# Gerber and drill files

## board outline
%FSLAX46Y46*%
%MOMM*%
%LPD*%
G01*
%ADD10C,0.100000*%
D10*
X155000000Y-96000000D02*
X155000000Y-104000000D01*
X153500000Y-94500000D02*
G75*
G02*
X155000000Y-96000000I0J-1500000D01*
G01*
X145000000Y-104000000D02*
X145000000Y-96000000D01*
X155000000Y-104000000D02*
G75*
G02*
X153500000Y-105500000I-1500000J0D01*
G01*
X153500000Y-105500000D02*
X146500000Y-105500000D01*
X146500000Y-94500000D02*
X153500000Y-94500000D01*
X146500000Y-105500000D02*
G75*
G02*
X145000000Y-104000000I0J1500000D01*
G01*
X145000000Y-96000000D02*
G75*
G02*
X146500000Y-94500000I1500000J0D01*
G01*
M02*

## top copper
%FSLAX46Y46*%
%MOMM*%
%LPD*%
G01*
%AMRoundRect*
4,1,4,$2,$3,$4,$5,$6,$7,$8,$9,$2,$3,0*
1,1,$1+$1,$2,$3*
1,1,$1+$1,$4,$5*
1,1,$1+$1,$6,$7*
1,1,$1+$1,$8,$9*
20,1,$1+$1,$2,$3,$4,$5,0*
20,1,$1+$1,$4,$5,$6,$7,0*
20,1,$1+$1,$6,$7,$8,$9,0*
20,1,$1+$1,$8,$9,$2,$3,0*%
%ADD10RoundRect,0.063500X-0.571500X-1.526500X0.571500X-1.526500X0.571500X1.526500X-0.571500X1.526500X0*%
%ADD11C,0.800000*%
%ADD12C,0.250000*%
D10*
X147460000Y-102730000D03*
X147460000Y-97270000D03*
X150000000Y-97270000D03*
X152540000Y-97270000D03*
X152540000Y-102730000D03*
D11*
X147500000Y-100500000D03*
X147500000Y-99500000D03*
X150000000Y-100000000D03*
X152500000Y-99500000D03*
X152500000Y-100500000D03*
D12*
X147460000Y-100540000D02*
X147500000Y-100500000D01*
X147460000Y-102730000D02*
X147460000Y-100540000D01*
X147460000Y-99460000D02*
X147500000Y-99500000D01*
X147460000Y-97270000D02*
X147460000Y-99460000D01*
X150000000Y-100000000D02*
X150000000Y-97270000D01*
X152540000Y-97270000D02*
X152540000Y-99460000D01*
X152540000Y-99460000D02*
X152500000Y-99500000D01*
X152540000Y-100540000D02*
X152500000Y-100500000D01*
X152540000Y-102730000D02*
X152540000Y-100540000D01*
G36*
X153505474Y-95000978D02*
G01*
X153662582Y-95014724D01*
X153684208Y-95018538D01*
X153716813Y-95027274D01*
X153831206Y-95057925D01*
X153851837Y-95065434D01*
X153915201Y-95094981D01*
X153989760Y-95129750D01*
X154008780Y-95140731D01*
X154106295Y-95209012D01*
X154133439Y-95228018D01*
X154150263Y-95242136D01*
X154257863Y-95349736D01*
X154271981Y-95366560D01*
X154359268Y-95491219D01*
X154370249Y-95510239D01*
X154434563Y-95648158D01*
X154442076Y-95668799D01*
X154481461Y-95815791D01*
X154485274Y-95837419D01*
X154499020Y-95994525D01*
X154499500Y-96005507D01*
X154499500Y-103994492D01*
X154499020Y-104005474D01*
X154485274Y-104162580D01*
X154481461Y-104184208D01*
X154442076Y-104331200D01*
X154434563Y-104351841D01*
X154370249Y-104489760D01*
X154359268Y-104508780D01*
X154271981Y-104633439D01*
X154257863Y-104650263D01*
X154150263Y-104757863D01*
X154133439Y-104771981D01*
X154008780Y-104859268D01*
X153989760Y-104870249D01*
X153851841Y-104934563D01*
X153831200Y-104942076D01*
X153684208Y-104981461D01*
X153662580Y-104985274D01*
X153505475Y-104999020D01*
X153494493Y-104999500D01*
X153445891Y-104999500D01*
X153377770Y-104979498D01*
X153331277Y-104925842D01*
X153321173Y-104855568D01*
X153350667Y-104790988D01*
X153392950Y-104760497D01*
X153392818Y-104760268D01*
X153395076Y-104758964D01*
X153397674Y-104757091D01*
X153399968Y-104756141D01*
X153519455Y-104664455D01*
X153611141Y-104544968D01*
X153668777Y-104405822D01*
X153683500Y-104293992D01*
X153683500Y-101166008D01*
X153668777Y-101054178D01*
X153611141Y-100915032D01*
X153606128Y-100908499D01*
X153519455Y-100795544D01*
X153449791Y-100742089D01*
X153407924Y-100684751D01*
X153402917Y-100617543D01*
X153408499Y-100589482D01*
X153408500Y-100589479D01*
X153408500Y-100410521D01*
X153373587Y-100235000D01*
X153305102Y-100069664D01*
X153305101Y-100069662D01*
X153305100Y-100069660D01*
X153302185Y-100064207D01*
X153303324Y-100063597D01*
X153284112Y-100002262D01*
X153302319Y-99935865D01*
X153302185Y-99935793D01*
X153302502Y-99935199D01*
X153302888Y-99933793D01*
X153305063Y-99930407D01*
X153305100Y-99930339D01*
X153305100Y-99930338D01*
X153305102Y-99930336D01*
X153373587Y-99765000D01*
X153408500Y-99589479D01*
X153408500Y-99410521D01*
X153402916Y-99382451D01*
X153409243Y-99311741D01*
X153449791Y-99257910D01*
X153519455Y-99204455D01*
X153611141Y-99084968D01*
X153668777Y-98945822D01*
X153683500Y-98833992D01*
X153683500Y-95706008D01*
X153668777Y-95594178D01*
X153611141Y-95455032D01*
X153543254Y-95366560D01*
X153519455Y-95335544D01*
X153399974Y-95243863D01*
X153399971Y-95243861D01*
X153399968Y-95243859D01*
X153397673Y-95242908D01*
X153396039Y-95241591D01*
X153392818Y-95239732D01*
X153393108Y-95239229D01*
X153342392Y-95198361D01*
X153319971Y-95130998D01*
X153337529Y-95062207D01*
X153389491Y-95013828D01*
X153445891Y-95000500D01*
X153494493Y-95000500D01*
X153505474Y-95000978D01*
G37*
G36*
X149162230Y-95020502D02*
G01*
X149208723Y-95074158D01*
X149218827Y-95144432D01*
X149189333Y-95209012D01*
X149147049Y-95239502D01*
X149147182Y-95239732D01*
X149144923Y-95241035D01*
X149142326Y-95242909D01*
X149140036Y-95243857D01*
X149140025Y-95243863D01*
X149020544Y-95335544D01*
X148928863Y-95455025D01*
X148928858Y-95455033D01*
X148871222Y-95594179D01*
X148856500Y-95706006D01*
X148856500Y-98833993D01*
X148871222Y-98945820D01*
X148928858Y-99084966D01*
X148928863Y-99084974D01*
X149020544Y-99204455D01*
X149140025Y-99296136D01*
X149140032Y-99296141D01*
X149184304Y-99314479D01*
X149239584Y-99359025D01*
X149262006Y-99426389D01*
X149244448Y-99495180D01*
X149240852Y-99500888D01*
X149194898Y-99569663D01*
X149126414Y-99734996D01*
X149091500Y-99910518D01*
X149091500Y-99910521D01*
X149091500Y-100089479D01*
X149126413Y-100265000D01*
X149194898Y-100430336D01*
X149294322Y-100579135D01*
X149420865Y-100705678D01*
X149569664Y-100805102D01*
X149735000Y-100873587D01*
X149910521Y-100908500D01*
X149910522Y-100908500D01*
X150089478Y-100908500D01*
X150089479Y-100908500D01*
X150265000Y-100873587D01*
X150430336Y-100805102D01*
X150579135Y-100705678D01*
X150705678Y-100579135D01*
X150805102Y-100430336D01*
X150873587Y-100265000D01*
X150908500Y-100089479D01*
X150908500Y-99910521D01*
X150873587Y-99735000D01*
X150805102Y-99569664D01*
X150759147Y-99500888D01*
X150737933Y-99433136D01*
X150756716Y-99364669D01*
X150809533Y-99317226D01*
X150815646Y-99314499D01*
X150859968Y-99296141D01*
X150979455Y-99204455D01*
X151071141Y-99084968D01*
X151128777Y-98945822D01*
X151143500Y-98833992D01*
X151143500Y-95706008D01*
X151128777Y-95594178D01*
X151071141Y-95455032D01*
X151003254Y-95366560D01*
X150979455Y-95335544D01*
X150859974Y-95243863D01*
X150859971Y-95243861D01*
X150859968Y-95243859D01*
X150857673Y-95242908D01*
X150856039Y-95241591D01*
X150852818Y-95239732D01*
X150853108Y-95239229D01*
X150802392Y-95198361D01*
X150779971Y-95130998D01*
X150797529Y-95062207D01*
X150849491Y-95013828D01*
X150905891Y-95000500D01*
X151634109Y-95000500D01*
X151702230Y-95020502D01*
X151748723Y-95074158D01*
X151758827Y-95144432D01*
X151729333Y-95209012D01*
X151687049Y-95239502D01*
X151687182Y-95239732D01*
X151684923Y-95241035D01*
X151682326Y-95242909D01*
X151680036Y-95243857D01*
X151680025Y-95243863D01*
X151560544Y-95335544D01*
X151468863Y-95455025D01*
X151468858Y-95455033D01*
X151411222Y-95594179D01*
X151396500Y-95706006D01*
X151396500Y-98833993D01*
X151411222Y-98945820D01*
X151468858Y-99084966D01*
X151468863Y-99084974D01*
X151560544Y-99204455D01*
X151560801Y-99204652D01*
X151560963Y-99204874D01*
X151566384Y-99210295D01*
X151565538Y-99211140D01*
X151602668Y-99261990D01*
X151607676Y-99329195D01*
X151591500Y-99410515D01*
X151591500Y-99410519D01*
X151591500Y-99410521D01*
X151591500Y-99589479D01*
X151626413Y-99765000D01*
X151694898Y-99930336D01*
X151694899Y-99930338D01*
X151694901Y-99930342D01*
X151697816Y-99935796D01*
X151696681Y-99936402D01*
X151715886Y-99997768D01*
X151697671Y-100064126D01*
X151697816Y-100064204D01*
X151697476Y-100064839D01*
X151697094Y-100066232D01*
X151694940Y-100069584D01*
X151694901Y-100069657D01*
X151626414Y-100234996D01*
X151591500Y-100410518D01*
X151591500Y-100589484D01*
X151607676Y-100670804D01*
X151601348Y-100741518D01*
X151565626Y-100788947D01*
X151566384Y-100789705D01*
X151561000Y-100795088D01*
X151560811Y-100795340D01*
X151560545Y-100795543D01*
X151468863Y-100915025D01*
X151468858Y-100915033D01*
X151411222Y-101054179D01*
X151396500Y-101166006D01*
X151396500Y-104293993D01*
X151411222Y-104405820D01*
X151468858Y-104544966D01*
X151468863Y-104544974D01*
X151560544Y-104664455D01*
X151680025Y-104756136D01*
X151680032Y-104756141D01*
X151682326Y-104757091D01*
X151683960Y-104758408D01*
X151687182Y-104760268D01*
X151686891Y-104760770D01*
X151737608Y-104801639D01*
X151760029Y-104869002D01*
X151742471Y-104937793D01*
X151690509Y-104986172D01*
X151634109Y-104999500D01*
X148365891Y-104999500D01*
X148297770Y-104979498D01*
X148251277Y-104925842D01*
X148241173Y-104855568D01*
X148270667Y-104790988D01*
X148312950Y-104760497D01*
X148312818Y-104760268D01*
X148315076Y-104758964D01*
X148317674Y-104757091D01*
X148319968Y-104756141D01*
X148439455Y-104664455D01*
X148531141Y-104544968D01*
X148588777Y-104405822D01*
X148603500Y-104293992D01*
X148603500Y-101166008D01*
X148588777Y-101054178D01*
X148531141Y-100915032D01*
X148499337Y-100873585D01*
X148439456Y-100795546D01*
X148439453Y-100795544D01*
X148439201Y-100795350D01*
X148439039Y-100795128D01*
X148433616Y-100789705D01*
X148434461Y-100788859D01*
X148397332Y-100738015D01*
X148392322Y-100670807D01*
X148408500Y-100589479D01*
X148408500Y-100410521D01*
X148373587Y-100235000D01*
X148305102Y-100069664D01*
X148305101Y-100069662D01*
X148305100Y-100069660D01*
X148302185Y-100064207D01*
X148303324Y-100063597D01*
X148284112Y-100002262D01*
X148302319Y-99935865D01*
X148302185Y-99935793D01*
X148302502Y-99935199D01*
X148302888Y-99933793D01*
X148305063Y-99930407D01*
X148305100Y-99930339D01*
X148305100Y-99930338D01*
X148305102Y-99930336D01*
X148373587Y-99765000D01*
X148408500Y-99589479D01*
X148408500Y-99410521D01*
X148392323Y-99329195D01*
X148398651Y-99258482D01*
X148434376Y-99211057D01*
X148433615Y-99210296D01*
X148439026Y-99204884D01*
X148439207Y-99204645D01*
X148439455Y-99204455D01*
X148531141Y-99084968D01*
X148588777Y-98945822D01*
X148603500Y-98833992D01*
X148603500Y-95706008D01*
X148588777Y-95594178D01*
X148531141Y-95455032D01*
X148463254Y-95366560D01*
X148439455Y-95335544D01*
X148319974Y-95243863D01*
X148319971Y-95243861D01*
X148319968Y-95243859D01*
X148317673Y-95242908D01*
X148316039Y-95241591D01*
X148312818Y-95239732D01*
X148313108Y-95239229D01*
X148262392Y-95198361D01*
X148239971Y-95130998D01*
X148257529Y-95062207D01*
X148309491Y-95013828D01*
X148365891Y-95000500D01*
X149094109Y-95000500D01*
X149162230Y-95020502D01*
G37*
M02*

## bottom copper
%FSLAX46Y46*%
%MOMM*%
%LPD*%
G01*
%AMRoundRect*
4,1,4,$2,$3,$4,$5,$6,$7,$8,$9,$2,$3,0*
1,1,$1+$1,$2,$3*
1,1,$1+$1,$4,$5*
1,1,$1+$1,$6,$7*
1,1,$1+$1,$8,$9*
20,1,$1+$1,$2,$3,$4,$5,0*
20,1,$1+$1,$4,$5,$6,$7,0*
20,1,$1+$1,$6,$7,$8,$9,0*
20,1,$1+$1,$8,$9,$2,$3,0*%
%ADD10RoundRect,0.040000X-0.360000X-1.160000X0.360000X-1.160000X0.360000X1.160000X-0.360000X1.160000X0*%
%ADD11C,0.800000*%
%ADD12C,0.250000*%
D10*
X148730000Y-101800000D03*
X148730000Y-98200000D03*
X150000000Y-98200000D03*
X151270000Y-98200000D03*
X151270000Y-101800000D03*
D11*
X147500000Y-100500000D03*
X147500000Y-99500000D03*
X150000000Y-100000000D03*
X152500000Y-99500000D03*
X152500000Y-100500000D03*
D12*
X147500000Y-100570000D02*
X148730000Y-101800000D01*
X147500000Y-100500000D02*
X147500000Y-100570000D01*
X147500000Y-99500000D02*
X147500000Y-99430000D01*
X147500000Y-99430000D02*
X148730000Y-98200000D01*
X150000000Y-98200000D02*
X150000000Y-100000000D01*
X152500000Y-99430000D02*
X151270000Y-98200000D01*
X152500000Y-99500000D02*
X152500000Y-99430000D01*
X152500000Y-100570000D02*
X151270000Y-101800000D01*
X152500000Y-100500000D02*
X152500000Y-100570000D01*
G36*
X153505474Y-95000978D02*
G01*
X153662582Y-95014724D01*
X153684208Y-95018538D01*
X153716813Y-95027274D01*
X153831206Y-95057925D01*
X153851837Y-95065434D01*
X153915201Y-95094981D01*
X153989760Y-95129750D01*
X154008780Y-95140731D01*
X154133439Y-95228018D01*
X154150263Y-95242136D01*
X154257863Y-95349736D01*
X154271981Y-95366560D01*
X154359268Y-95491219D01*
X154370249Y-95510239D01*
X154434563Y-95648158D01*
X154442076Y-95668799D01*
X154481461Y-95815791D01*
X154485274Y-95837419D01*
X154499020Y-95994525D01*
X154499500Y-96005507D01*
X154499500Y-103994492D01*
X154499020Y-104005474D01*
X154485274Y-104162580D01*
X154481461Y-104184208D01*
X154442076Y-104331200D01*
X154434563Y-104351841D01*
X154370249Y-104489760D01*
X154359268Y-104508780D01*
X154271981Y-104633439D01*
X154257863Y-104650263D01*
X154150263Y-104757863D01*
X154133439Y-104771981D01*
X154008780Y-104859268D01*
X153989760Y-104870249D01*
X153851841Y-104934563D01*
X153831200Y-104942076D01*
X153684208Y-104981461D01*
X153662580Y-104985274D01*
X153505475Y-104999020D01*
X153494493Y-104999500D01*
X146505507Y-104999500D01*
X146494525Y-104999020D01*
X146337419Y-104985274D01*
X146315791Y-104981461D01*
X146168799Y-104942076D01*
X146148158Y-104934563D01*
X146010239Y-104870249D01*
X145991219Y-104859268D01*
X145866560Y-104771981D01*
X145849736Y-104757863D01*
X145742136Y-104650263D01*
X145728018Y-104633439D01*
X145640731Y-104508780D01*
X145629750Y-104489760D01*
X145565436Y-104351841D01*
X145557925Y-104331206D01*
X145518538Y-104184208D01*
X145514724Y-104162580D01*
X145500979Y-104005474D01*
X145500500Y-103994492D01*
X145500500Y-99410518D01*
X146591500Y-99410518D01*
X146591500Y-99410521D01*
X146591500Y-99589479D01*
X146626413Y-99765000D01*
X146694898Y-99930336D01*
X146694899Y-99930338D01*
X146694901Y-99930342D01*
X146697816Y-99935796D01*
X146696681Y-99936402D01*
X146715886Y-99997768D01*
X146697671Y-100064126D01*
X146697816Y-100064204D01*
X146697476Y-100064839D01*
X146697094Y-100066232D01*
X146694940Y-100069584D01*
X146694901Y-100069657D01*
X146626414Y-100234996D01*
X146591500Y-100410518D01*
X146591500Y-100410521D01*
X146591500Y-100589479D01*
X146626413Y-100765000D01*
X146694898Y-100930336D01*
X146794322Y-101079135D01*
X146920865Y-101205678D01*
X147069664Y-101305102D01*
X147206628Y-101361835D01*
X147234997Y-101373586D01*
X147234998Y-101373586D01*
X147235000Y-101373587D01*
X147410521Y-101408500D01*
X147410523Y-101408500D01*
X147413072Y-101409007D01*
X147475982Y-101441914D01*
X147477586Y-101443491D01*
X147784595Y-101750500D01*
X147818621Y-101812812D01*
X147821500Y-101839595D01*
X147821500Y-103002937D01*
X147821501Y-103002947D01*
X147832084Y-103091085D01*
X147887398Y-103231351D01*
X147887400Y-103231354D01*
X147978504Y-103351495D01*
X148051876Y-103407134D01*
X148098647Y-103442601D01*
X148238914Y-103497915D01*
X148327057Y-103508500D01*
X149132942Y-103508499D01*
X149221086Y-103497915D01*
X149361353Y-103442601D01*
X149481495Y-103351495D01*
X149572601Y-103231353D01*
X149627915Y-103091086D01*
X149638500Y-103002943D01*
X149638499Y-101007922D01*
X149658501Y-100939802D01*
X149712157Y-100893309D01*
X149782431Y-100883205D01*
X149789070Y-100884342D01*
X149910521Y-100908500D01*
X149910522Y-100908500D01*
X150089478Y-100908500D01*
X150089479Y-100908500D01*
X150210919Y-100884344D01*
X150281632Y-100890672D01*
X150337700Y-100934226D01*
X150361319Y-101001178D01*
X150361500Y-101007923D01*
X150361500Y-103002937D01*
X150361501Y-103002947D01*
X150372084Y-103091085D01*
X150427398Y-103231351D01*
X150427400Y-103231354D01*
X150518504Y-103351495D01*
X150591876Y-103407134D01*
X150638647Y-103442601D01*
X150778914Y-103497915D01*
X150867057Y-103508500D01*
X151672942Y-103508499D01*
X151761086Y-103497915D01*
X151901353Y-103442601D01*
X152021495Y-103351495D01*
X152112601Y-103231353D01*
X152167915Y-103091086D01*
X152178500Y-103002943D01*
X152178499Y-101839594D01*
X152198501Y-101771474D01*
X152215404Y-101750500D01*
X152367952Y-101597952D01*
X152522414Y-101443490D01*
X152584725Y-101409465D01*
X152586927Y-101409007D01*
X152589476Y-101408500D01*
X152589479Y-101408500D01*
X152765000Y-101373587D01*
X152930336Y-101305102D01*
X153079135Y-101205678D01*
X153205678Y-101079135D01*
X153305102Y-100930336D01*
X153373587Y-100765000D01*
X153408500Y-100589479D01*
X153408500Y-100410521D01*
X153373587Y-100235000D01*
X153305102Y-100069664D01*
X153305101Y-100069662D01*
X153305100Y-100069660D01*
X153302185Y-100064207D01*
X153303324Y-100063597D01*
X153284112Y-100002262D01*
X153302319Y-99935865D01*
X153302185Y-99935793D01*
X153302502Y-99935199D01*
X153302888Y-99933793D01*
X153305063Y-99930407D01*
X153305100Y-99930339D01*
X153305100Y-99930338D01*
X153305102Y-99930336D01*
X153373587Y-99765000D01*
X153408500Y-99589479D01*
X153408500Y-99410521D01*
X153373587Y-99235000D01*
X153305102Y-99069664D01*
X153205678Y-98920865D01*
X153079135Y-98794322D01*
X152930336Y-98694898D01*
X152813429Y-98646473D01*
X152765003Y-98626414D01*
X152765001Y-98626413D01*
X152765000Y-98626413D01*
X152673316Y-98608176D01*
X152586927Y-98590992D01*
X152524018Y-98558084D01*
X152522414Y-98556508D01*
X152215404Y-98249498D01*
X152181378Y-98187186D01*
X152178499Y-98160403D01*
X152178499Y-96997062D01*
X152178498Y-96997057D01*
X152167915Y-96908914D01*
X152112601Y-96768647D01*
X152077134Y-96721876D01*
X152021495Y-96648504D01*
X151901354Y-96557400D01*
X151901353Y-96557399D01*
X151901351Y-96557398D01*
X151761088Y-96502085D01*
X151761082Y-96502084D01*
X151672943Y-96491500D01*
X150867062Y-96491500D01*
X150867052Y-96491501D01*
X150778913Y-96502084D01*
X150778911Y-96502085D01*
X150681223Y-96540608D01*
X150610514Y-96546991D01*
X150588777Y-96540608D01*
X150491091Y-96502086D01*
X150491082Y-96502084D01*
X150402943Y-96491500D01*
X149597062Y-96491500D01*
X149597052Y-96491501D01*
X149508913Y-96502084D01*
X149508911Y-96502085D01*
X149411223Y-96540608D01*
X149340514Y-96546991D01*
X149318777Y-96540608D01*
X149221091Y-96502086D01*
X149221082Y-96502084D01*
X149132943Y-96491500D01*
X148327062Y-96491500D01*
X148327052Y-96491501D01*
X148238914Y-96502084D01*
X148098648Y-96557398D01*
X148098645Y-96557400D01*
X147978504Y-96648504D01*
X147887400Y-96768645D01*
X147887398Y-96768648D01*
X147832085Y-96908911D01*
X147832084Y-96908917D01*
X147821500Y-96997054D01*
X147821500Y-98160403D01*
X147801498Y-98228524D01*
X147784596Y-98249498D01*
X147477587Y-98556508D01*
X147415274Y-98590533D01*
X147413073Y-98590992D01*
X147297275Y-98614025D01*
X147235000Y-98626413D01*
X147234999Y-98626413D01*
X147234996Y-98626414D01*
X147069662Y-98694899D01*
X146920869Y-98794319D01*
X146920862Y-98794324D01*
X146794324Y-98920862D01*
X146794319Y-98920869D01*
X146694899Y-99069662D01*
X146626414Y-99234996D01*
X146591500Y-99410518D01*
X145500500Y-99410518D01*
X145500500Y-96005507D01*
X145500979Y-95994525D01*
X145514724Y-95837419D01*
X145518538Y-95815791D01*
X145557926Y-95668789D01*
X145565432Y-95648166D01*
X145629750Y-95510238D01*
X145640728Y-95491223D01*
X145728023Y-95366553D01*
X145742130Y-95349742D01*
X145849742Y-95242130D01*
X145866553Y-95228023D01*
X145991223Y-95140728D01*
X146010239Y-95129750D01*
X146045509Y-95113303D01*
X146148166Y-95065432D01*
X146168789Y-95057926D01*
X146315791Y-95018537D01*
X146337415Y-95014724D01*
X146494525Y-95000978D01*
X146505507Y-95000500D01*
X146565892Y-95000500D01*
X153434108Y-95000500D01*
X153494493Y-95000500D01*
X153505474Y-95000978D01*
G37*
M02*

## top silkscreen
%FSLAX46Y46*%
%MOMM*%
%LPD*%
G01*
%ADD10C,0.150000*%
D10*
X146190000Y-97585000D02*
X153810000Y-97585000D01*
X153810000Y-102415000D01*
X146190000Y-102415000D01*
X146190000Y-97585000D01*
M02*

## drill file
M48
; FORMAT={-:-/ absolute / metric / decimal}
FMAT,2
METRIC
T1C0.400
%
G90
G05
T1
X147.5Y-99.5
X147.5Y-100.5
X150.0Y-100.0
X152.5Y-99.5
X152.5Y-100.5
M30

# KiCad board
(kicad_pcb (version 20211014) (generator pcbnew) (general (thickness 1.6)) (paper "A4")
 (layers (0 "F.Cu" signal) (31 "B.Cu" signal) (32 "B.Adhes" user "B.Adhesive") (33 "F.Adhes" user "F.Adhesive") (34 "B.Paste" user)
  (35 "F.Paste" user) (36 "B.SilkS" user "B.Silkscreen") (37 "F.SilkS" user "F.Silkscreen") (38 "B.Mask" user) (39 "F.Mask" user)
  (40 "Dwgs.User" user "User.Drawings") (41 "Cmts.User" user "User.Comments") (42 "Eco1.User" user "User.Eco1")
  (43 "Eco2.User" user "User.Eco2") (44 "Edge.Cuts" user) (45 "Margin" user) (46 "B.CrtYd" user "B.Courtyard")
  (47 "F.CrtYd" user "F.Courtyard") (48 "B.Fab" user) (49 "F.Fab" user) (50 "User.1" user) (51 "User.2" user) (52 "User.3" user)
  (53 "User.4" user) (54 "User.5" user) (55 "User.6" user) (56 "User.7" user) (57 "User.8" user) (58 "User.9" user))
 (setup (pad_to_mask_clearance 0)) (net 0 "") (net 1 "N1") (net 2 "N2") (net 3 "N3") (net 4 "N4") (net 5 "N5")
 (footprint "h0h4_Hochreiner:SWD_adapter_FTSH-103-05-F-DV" (layer "F.Cu") (at 150 100)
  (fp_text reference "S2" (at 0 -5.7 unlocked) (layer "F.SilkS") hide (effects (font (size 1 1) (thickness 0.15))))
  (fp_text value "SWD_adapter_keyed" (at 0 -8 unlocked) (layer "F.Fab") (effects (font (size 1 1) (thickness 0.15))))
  (pad "1" smd roundrect (at -1.27 1.8) (size 0.8 2.4) (layers "B.Cu" "B.Paste" "B.Mask") (roundrect_rratio 0.05) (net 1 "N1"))
  (pad "2" smd roundrect (at -1.27 -1.8) (size 0.8 2.4) (layers "B.Cu" "B.Paste" "B.Mask") (roundrect_rratio 0.05) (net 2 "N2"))
  (pad "3" smd roundrect (at 0 -1.8) (size 0.8 2.4) (layers "B.Cu" "B.Paste" "B.Mask") (roundrect_rratio 0.05) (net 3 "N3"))
  (pad "4" smd roundrect (at 1.27 -1.8) (size 0.8 2.4) (layers "B.Cu" "B.Paste" "B.Mask") (roundrect_rratio 0.05) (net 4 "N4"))
  (pad "5" smd roundrect (at 1.27 1.8) (size 0.8 2.4) (layers "B.Cu" "B.Paste" "B.Mask") (roundrect_rratio 0.05) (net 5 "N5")))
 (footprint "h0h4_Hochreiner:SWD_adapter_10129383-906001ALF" (layer "F.Cu") (at 150 100)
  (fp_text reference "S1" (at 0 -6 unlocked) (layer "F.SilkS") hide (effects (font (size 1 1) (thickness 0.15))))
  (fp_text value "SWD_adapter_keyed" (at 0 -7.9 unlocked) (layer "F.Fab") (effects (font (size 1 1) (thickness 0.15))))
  (fp_rect (start -3.81 -2.415) (end 3.81 2.415) (layer "F.SilkS") (width 0.15) (fill none))
  (pad "1" smd roundrect (at -2.54 2.73) (size 1.27 3.18) (layers "F.Cu" "F.Paste" "F.Mask") (roundrect_rratio 0.05) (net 1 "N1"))
  (pad "2" smd roundrect (at -2.54 -2.73) (size 1.27 3.18) (layers "F.Cu" "F.Paste" "F.Mask") (roundrect_rratio 0.05) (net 2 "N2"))
  (pad "3" smd roundrect (at 0 -2.73) (size 1.27 3.18) (layers "F.Cu" "F.Paste" "F.Mask") (roundrect_rratio 0.05) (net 3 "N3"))
  (pad "4" smd roundrect (at 2.54 -2.73) (size 1.27 3.18) (layers "F.Cu" "F.Paste" "F.Mask") (roundrect_rratio 0.05) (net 4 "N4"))
  (pad "5" smd roundrect (at 2.54 2.73) (size 1.27 3.18) (layers "F.Cu" "F.Paste" "F.Mask") (roundrect_rratio 0.05) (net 5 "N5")))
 (gr_line (start 155 96) (end 155 104) (layer "Edge.Cuts") (width 0.1))
 (gr_arc (start 153.5 94.5) (mid 154.56066 94.93934) (end 155 96) (layer "Edge.Cuts") (width 0.1))
 (gr_line (start 145 104) (end 145 96) (layer "Edge.Cuts") (width 0.1))
 (gr_arc (start 155 104) (mid 154.56066 105.06066) (end 153.5 105.5) (layer "Edge.Cuts") (width 0.1))
 (gr_line (start 153.5 105.5) (end 146.5 105.5) (layer "Edge.Cuts") (width 0.1))
 (gr_line (start 146.5 94.5) (end 153.5 94.5) (layer "Edge.Cuts") (width 0.1))
 (gr_arc (start 146.5 105.5) (mid 145.43934 105.06066) (end 145 104) (layer "Edge.Cuts") (width 0.1))
 (gr_arc (start 145 96) (mid 145.43934 94.93934) (end 146.5 94.5) (layer "Edge.Cuts") (width 0.1))
 (segment (start 147.46 100.54) (end 147.5 100.5) (width 0.25) (layer "F.Cu") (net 1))
 (segment (start 147.46 102.73) (end 147.46 100.54) (width 0.25) (layer "F.Cu") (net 1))
 (via (at 147.5 100.5) (size 0.8) (drill 0.4) (layers "F.Cu" "B.Cu") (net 1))
 (segment (start 147.5 100.57) (end 148.73 101.8) (width 0.25) (layer "B.Cu") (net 1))
 (segment (start 147.5 100.5) (end 147.5 100.57) (width 0.25) (layer "B.Cu") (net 1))
 (segment (start 147.46 99.46) (end 147.5 99.5) (width 0.25) (layer "F.Cu") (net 2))
 (segment (start 147.46 97.27) (end 147.46 99.46) (width 0.25) (layer "F.Cu") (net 2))
 (via (at 147.5 99.5) (size 0.8) (drill 0.4) (layers "F.Cu" "B.Cu") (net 2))
 (segment (start 147.5 99.5) (end 147.5 99.43) (width 0.25) (layer "B.Cu") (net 2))
 (segment (start 147.5 99.43) (end 148.73 98.2) (width 0.25) (layer "B.Cu") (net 2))
 (segment (start 150 100) (end 150 97.27) (width 0.25) (layer "F.Cu") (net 3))
 (via (at 150 100) (size 0.8) (drill 0.4) (layers "F.Cu" "B.Cu") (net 3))
 (segment (start 150 98.2) (end 150 100) (width 0.25) (layer "B.Cu") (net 3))
 (segment (start 152.54 97.27) (end 152.54 99.46) (width 0.25) (layer "F.Cu") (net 4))
 (segment (start 152.54 99.46) (end 152.5 99.5) (width 0.25) (layer "F.Cu") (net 4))
 (via (at 152.5 99.5) (size 0.8) (drill 0.4) (layers "F.Cu" "B.Cu") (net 4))
 (segment (start 152.5 99.43) (end 151.27 98.2) (width 0.25) (layer "B.Cu") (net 4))
 (segment (start 152.5 99.5) (end 152.5 99.43) (width 0.25) (layer "B.Cu") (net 4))
 (segment (start 152.54 100.54) (end 152.5 100.5) (width 0.25) (layer "F.Cu") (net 5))
 (segment (start 152.54 102.73) (end 152.54 100.54) (width 0.25) (layer "F.Cu") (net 5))
 (via (at 152.5 100.5) (size 0.8) (drill 0.4) (layers "F.Cu" "B.Cu") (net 5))
 (segment (start 152.5 100.57) (end 151.27 101.8) (width 0.25) (layer "B.Cu") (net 5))
 (segment (start 152.5 100.5) (end 152.5 100.57) (width 0.25) (layer "B.Cu") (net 5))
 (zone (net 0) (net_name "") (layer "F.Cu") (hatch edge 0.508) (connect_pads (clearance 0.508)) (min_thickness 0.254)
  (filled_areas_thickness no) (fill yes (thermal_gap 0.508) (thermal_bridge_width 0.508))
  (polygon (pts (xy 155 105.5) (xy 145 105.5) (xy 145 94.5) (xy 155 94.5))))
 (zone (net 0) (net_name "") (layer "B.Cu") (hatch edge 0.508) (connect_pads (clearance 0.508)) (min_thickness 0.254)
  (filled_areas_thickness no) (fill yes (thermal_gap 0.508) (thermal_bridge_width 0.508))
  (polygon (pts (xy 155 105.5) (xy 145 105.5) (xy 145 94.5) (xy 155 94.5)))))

